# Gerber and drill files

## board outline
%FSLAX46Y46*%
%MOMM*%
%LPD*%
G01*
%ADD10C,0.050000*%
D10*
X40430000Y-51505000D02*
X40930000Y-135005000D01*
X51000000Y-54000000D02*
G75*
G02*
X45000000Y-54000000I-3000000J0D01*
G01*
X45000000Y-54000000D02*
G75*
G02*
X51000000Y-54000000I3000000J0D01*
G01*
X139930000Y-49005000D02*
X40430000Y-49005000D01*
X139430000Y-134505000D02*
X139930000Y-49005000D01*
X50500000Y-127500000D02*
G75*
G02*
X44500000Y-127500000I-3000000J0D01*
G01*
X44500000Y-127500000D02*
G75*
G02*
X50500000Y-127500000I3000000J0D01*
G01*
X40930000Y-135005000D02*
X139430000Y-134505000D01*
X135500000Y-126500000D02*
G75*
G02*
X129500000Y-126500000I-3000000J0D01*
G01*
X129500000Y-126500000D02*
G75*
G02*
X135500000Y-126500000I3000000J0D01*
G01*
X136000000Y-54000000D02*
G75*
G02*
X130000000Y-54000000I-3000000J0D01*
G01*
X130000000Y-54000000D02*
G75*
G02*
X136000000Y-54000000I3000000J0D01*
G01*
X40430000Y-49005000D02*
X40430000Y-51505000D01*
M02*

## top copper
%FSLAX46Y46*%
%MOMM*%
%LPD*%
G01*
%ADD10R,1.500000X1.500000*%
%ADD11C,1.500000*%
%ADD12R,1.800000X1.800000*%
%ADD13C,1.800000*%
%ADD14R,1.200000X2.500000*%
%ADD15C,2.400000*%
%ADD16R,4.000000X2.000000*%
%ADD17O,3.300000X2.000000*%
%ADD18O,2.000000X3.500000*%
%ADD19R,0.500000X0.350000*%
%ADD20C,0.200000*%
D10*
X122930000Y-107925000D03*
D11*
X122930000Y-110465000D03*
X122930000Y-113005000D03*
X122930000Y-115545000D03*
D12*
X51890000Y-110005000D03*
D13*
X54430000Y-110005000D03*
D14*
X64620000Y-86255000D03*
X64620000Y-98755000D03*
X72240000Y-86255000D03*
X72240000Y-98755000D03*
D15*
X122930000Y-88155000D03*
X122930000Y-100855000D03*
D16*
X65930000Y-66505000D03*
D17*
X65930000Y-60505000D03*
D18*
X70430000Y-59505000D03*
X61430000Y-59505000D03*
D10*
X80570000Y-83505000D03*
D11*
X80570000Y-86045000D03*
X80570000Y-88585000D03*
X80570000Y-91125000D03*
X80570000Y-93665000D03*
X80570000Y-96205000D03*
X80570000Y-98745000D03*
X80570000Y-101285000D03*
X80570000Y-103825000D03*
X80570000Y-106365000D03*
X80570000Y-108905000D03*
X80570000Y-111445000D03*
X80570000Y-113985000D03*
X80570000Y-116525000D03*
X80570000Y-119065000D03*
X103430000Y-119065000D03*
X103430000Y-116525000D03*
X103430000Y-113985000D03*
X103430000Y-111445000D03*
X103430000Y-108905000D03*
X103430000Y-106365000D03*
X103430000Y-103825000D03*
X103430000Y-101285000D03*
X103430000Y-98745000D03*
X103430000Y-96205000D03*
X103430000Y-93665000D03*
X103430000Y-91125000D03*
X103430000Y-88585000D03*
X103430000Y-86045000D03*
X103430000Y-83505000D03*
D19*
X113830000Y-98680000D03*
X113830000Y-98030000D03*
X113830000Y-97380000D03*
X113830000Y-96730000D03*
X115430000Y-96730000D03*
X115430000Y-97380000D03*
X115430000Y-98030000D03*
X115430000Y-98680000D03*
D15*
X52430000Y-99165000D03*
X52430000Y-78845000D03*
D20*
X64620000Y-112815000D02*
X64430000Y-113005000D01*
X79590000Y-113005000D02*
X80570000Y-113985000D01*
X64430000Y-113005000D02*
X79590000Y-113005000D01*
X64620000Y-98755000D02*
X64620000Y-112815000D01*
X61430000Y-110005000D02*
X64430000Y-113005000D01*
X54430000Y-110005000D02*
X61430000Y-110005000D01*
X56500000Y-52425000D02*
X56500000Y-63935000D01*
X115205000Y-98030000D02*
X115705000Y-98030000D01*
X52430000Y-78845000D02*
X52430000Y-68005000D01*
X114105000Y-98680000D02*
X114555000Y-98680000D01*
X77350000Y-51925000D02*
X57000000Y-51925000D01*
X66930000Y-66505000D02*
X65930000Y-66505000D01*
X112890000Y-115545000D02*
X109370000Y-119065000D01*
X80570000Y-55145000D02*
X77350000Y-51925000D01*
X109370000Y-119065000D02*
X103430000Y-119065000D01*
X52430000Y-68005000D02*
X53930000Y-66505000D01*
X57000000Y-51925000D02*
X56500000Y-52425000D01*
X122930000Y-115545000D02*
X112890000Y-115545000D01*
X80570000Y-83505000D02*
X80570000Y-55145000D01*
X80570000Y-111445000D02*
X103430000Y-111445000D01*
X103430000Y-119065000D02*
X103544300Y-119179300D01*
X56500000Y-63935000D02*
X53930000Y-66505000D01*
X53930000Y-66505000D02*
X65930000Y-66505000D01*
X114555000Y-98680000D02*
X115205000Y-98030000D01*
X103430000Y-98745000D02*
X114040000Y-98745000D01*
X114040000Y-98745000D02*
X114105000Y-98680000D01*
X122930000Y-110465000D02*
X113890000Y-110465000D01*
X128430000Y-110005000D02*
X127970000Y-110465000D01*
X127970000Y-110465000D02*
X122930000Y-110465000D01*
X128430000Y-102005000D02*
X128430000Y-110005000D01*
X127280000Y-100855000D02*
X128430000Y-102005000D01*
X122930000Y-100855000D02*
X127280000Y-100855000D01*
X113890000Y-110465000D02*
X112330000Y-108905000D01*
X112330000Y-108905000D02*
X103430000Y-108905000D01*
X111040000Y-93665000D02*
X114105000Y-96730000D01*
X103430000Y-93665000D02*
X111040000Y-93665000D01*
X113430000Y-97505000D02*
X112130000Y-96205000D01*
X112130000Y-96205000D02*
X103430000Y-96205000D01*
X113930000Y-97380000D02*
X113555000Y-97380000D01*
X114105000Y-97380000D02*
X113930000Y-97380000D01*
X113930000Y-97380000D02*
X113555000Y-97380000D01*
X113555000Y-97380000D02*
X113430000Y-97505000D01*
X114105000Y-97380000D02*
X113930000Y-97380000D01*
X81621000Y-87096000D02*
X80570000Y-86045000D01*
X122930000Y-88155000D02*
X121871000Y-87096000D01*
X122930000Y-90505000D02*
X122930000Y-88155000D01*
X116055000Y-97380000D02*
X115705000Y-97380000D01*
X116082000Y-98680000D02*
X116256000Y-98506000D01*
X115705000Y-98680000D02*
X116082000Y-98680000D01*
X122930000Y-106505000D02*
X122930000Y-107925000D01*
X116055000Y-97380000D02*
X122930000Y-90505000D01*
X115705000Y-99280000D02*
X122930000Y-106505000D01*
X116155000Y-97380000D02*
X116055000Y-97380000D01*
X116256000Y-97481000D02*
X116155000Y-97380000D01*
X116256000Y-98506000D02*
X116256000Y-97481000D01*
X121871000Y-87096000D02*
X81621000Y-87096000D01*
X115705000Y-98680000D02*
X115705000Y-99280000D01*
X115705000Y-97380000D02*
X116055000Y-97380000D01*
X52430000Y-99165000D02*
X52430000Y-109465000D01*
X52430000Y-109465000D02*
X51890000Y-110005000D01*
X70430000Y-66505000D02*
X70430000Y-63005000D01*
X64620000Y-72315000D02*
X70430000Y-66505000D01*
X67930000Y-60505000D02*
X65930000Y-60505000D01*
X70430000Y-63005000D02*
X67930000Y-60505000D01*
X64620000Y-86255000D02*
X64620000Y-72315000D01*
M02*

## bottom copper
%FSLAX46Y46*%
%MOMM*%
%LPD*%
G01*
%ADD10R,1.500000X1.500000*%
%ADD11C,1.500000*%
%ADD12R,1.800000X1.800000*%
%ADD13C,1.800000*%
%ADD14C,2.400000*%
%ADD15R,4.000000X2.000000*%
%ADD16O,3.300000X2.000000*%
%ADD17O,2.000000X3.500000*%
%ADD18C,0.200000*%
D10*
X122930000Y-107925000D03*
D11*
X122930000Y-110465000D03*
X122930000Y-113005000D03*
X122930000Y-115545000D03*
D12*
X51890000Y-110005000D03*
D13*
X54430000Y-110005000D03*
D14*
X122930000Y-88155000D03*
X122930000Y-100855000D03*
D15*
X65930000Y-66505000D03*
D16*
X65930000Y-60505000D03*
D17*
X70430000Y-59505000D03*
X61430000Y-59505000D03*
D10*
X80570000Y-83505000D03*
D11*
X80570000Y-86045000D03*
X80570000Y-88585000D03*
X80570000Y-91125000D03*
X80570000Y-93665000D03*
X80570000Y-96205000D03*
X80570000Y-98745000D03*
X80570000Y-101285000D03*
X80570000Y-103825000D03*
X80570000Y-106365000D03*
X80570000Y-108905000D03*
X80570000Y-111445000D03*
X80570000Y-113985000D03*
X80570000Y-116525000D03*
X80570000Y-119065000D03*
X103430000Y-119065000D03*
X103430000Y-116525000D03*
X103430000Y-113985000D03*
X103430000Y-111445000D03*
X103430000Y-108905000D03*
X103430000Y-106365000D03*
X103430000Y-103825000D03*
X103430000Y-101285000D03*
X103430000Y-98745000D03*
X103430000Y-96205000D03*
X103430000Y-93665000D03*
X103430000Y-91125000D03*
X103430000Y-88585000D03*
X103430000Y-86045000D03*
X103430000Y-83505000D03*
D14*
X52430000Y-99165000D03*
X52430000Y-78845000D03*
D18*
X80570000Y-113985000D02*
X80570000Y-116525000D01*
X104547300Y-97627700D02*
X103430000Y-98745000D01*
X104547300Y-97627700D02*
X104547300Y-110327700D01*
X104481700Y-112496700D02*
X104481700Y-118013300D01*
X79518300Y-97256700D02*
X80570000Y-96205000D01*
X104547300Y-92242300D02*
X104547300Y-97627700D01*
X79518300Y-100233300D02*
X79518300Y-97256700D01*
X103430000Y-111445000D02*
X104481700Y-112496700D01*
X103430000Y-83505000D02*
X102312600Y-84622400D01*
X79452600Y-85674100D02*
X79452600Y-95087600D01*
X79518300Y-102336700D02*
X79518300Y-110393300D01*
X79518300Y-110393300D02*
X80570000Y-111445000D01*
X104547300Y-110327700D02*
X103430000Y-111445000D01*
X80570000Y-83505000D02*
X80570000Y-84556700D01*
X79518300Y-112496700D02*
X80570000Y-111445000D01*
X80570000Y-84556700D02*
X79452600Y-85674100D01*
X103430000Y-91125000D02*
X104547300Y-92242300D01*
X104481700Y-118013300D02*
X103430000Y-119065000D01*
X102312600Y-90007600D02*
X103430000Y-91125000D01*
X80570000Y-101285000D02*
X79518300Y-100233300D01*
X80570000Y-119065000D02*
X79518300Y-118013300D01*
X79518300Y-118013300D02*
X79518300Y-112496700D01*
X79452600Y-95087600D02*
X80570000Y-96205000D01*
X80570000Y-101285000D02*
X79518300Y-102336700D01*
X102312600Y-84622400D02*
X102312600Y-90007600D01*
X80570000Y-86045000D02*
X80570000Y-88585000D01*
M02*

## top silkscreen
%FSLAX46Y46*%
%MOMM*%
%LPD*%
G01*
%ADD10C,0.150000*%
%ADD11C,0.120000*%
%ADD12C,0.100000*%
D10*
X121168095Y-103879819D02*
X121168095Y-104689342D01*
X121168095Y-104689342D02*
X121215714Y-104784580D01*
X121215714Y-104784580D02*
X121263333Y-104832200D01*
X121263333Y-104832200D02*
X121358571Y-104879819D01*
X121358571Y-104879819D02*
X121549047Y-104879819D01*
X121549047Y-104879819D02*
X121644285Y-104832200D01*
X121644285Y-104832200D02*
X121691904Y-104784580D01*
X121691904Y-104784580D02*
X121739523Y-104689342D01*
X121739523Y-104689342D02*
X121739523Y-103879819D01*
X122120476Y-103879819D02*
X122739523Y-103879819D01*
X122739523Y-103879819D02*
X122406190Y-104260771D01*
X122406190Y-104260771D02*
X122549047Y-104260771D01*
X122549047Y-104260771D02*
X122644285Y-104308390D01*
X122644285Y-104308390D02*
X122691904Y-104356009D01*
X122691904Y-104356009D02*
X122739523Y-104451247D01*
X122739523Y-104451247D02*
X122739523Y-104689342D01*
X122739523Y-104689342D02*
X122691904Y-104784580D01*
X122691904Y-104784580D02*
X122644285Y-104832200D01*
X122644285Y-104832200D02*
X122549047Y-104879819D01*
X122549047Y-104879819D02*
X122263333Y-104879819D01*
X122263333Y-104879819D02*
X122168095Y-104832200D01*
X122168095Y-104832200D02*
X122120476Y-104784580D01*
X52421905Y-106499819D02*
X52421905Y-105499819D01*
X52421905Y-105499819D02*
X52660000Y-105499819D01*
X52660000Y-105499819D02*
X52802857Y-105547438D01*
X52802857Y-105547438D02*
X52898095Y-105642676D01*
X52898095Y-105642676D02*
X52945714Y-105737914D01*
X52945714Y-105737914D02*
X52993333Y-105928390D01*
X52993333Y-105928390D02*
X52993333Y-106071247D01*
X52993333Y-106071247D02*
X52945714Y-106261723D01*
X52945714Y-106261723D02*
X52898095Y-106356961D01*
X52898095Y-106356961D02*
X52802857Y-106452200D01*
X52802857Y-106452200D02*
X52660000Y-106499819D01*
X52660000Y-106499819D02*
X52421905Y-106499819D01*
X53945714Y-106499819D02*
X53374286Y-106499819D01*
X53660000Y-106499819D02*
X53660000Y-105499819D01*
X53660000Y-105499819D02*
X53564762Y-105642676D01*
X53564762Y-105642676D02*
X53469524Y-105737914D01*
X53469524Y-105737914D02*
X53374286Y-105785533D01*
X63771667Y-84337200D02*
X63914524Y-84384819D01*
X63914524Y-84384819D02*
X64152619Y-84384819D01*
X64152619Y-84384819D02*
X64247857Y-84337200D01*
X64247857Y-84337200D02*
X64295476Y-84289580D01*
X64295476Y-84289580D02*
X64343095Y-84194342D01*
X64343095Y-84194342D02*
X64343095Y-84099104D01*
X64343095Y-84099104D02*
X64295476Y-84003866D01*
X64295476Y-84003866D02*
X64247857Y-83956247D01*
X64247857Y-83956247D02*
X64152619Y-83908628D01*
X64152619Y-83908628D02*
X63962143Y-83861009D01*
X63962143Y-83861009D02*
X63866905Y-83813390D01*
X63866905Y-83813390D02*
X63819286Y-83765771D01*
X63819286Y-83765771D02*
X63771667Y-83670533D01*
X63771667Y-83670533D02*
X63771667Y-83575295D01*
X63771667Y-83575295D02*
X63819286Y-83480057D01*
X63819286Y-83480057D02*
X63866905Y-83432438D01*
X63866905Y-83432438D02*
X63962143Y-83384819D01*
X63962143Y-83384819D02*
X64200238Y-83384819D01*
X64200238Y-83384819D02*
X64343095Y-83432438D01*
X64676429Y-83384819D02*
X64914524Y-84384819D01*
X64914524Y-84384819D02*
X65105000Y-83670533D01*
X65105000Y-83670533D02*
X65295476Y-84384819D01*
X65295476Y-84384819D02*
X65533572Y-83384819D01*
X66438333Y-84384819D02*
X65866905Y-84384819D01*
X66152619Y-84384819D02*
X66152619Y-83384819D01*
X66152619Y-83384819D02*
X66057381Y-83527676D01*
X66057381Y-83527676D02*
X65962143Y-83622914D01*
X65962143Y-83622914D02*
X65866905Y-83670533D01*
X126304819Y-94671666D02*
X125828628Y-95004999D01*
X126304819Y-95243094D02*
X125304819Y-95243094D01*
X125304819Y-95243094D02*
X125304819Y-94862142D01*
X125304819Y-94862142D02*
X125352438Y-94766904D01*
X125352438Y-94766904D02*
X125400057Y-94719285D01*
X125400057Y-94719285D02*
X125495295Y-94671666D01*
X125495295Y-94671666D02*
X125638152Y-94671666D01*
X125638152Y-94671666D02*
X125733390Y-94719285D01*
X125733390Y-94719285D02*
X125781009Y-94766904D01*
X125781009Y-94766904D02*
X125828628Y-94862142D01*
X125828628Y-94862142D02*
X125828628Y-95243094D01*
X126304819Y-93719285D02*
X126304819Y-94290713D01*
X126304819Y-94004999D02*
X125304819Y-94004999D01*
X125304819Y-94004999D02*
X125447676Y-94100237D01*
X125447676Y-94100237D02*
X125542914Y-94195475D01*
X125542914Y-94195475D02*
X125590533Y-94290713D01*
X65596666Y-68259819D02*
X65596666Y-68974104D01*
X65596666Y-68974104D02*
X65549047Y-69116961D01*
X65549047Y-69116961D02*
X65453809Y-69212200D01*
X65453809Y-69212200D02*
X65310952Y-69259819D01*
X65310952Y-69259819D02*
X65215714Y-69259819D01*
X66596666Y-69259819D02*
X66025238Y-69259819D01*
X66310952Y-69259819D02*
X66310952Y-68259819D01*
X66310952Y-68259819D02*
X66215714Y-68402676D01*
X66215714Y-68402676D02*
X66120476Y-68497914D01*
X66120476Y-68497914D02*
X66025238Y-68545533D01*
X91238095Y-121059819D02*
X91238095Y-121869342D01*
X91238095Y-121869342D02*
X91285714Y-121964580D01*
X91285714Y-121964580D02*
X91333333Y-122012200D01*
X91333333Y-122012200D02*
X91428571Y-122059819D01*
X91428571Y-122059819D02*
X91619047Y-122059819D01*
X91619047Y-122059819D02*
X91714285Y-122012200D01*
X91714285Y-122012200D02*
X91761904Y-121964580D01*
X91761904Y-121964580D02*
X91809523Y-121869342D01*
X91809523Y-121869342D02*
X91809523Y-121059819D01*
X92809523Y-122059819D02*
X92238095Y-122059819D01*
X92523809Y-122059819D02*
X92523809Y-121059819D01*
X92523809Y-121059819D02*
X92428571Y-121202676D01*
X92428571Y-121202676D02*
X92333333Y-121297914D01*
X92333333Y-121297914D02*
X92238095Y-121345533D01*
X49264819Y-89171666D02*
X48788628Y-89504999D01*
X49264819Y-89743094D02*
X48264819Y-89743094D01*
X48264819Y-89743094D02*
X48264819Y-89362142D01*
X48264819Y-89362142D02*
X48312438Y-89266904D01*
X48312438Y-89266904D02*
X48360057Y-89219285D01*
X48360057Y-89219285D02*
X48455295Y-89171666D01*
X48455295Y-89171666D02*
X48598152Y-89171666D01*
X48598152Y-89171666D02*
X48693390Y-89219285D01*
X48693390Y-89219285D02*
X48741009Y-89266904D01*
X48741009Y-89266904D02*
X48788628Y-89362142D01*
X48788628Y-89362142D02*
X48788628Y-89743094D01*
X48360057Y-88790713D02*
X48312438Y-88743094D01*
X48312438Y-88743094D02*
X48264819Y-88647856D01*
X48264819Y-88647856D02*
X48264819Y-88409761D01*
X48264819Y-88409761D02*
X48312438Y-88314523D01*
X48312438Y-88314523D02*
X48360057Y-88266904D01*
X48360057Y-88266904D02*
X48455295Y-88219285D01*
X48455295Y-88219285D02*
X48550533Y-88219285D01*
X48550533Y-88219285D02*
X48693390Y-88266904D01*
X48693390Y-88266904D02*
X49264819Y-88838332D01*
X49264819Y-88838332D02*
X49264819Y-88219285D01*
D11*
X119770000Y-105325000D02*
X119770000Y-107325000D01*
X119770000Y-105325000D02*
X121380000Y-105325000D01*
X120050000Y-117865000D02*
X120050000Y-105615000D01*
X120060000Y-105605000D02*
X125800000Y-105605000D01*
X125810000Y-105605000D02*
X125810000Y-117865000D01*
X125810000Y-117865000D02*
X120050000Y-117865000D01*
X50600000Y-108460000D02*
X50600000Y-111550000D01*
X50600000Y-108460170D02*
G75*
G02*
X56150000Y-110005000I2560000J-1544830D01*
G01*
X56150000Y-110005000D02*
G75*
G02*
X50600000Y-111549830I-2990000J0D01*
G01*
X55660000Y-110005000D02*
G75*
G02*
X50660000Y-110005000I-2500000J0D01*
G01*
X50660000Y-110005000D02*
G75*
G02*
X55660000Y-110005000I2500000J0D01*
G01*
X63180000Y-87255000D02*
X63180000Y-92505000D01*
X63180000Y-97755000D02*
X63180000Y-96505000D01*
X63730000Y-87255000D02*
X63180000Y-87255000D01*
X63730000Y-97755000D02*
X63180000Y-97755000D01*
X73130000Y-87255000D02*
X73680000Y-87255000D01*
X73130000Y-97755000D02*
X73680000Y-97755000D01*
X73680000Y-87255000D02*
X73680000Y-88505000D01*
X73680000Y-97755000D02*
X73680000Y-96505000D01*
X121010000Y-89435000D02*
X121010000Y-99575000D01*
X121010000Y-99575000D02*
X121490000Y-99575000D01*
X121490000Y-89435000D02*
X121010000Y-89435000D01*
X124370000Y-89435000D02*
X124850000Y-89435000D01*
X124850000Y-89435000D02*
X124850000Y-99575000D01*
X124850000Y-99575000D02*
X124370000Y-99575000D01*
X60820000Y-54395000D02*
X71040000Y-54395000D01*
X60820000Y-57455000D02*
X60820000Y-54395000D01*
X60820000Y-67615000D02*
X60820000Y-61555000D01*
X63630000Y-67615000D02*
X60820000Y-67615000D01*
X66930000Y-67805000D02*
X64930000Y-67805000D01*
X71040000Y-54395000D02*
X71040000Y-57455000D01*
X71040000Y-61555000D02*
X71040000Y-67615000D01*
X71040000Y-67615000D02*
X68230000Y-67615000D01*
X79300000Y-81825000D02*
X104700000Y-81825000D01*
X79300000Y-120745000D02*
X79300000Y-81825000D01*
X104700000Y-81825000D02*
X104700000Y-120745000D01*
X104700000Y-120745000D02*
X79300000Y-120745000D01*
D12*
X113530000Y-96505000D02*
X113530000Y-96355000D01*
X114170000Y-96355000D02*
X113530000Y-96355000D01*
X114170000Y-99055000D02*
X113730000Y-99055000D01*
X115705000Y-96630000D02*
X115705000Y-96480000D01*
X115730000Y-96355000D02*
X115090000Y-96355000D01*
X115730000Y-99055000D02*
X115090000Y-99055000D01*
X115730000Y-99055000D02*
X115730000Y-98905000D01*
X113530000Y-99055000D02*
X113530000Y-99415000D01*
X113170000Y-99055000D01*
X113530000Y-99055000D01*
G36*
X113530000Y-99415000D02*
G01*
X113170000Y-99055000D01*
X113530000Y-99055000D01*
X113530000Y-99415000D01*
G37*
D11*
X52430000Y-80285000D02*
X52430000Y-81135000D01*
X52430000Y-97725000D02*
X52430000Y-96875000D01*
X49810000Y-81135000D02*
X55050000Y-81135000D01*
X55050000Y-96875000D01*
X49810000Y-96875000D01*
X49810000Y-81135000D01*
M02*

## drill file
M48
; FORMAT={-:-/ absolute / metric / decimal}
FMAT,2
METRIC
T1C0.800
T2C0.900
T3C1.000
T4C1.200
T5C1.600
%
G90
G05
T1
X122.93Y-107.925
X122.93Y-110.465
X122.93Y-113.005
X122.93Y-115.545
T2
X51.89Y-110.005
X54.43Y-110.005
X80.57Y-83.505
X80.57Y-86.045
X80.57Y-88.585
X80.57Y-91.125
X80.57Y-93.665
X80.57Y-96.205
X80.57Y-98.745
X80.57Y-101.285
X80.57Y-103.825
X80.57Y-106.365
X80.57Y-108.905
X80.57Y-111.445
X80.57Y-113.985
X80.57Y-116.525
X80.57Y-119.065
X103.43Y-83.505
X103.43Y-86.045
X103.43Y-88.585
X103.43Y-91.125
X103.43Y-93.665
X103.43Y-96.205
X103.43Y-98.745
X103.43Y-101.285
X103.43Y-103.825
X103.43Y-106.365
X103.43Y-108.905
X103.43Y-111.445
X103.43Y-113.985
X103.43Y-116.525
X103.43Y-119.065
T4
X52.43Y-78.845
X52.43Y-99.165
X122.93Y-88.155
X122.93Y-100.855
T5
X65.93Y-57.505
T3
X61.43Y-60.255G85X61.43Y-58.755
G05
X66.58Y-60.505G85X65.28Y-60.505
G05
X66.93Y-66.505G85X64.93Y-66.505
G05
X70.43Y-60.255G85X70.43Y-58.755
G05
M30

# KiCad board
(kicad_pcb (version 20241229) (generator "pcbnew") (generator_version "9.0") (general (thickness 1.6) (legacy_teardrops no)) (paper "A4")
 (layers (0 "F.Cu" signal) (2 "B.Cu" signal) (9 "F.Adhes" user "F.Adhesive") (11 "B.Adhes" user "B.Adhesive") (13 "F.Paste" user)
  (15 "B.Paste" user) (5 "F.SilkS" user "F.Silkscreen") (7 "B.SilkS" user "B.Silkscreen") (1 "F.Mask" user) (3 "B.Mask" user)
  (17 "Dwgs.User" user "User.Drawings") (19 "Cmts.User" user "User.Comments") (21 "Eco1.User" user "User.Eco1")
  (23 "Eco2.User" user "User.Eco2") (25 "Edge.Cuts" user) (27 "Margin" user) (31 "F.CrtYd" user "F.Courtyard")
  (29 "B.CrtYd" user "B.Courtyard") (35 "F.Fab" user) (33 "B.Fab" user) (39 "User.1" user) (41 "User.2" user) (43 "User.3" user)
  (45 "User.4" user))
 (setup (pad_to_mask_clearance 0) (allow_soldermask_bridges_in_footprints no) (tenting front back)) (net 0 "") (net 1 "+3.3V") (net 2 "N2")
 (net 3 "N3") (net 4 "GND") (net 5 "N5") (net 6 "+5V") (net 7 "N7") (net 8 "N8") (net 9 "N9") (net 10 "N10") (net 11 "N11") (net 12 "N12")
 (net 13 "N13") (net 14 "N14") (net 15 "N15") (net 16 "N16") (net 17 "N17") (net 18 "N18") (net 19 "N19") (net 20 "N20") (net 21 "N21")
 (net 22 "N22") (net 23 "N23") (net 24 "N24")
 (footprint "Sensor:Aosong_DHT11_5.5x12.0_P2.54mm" (layer "F.Cu") (at 122.93 107.925)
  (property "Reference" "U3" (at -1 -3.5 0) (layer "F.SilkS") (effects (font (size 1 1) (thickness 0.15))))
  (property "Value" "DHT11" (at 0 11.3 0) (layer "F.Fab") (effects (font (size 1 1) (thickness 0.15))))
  (fp_line (start -3.16 -2.6) (end -3.16 -0.6) (stroke (width 0.12) (type solid)) (layer "F.SilkS"))
  (fp_line (start -3.16 -2.6) (end -1.55 -2.6) (stroke (width 0.12) (type solid)) (layer "F.SilkS"))
  (fp_line (start -2.88 9.94) (end -2.88 -2.31) (stroke (width 0.12) (type solid)) (layer "F.SilkS"))
  (fp_line (start -2.87 -2.32) (end 2.87 -2.32) (stroke (width 0.12) (type solid)) (layer "F.SilkS"))
  (fp_line (start 2.88 -2.32) (end 2.88 9.94) (stroke (width 0.12) (type solid)) (layer "F.SilkS"))
  (fp_line (start 2.88 9.94) (end -2.88 9.94) (stroke (width 0.12) (type solid)) (layer "F.SilkS"))
  (pad "1" thru_hole rect (at 0 0) (size 1.5 1.5) (drill 0.8) (layers "*.Cu" "*.Mask") (remove_unused_layers no) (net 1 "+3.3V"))
  (pad "2" thru_hole circle (at 0 2.54) (size 1.5 1.5) (drill 0.8) (layers "*.Cu" "*.Mask") (remove_unused_layers no) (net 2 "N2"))
  (pad "3" thru_hole circle (at 0 5.08) (size 1.5 1.5) (drill 0.8) (layers "*.Cu" "*.Mask") (remove_unused_layers no) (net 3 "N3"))
  (pad "4" thru_hole circle (at 0 7.62) (size 1.5 1.5) (drill 0.8) (layers "*.Cu" "*.Mask") (remove_unused_layers no) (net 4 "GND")))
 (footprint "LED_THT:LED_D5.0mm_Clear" (layer "F.Cu") (at 51.89 110.005)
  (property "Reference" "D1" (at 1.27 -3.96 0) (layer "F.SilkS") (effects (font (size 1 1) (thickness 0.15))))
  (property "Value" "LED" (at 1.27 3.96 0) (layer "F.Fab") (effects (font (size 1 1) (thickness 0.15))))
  (fp_line (start -1.29 -1.545) (end -1.29 1.545) (stroke (width 0.12) (type solid)) (layer "F.SilkS"))
  (fp_arc (start -1.29 -1.54483) (mid 2.071779 -2.880495) (end 4.26 0) (stroke (width 0.12) (type solid)) (layer "F.SilkS"))
  (fp_arc (start 4.26 0) (mid 2.071779 2.880495) (end -1.29 1.54483) (stroke (width 0.12) (type solid)) (layer "F.SilkS"))
  (fp_circle (center 1.27 0) (end 3.77 0) (stroke (width 0.12) (type solid)) (fill no) (layer "F.SilkS"))
  (pad "1" thru_hole rect (at 0 0) (size 1.8 1.8) (drill 0.9) (layers "*.Cu" "*.Mask") (remove_unused_layers no) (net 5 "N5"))
  (pad "2" thru_hole circle (at 2.54 0) (size 1.8 1.8) (drill 0.9) (layers "*.Cu" "*.Mask") (remove_unused_layers no) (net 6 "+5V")))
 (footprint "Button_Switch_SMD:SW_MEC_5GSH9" (layer "F.Cu") (at 68.43 92.505)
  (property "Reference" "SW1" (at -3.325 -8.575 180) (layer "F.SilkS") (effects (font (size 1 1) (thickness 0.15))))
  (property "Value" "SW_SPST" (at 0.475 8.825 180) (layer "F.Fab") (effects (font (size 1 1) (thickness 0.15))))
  (fp_line (start -5.25 -5.25) (end -5.25 0) (stroke (width 0.12) (type solid)) (layer "F.SilkS"))
  (fp_line (start -5.25 5.25) (end -5.25 4) (stroke (width 0.12) (type solid)) (layer "F.SilkS"))
  (fp_line (start -4.7 -5.25) (end -5.25 -5.25) (stroke (width 0.12) (type solid)) (layer "F.SilkS"))
  (fp_line (start -4.7 5.25) (end -5.25 5.25) (stroke (width 0.12) (type solid)) (layer "F.SilkS"))
  (fp_line (start 4.7 -5.25) (end 5.25 -5.25) (stroke (width 0.12) (type solid)) (layer "F.SilkS"))
  (fp_line (start 4.7 5.25) (end 5.25 5.25) (stroke (width 0.12) (type solid)) (layer "F.SilkS"))
  (fp_line (start 5.25 -5.25) (end 5.25 -4) (stroke (width 0.12) (type solid)) (layer "F.SilkS"))
  (fp_line (start 5.25 5.25) (end 5.25 4) (stroke (width 0.12) (type solid)) (layer "F.SilkS"))
  (pad "1" smd rect (at -3.81 -6.25 90) (size 2.5 1.2) (layers "F.Cu" "F.Mask" "F.Paste") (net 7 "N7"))
  (pad "2" smd rect (at -3.81 6.25 90) (size 2.5 1.2) (layers "F.Cu" "F.Mask" "F.Paste") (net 6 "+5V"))
  (pad "3" smd rect (at 3.81 -6.25 90) (size 2.5 1.2) (layers "F.Cu" "F.Mask" "F.Paste"))
  (pad "4" smd rect (at 3.81 6.25 90) (size 2.5 1.2) (layers "F.Cu" "F.Mask" "F.Paste")))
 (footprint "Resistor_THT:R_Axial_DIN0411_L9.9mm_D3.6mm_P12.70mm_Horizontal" (layer "F.Cu") (at 122.93 88.155 -90)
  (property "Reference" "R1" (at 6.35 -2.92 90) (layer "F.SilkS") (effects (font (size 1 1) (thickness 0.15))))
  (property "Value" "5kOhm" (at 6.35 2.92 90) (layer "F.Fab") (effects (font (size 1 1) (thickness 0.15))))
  (fp_line (start 1.28 1.92) (end 11.42 1.92) (stroke (width 0.12) (type solid)) (layer "F.SilkS"))
  (fp_line (start 11.42 1.92) (end 11.42 1.44) (stroke (width 0.12) (type solid)) (layer "F.SilkS"))
  (fp_line (start 1.28 1.44) (end 1.28 1.92) (stroke (width 0.12) (type solid)) (layer "F.SilkS"))
  (fp_line (start 1.28 -1.44) (end 1.28 -1.92) (stroke (width 0.12) (type solid)) (layer "F.SilkS"))
  (fp_line (start 1.28 -1.92) (end 11.42 -1.92) (stroke (width 0.12) (type solid)) (layer "F.SilkS"))
  (fp_line (start 11.42 -1.92) (end 11.42 -1.44) (stroke (width 0.12) (type solid)) (layer "F.SilkS"))
  (pad "1" thru_hole circle (at 0 0 270) (size 2.4 2.4) (drill 1.2) (layers "*.Cu" "*.Mask") (remove_unused_layers no) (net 1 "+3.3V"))
  (pad "2" thru_hole circle (at 12.7 0 270) (size 2.4 2.4) (drill 1.2) (layers "*.Cu" "*.Mask") (remove_unused_layers no) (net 2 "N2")))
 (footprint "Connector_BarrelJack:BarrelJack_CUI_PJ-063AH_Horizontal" (layer "F.Cu") (at 65.93 66.505 180)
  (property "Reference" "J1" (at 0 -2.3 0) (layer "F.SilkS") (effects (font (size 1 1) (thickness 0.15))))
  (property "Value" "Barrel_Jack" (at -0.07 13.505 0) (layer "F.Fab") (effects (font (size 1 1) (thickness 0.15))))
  (fp_line (start 5.11 12.11) (end -5.11 12.11) (stroke (width 0.12) (type solid)) (layer "F.SilkS"))
  (fp_line (start 5.11 9.05) (end 5.11 12.11) (stroke (width 0.12) (type solid)) (layer "F.SilkS"))
  (fp_line (start 5.11 -1.11) (end 5.11 4.95) (stroke (width 0.12) (type solid)) (layer "F.SilkS"))
  (fp_line (start 2.3 -1.11) (end 5.11 -1.11) (stroke (width 0.12) (type solid)) (layer "F.SilkS"))
  (fp_line (start -1 -1.3) (end 1 -1.3) (stroke (width 0.12) (type solid)) (layer "F.SilkS"))
  (fp_line (start -5.11 12.11) (end -5.11 9.05) (stroke (width 0.12) (type solid)) (layer "F.SilkS"))
  (fp_line (start -5.11 4.95) (end -5.11 -1.11) (stroke (width 0.12) (type solid)) (layer "F.SilkS"))
  (fp_line (start -5.11 -1.11) (end -2.3 -1.11) (stroke (width 0.12) (type solid)) (layer "F.SilkS"))
  (pad "" np_thru_hole circle (at 0 9 180) (size 1.6 1.6) (drill 1.6) (layers "*.Cu" "*.Mask"))
  (pad "1" thru_hole rect (at 0 0 180) (size 4 2) (drill oval 3 1) (layers "*.Cu" "*.Mask") (remove_unused_layers no) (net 4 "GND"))
  (pad "2" thru_hole oval (at 0 6 180) (size 3.3 2) (drill oval 2.3 1) (layers "*.Cu" "*.Mask") (remove_unused_layers no) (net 7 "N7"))
  (pad "MP" thru_hole oval (at -4.5 7 180) (size 2 3.5) (drill oval 1 2.5) (layers "*.Cu" "*.Mask") (remove_unused_layers no))
  (pad "MP" thru_hole oval (at 4.5 7 180) (size 2 3.5) (drill oval 1 2.5) (layers "*.Cu" "*.Mask") (remove_unused_layers no)))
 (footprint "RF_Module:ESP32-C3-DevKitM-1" (layer "F.Cu") (at 80.57 83.505)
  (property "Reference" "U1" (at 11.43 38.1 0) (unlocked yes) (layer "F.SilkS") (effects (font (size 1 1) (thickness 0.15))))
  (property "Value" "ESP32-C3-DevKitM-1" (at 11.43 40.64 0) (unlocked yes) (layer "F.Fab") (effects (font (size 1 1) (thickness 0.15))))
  (fp_line (start -1.27 -1.68) (end 24.13 -1.68) (stroke (width 0.12) (type solid)) (layer "F.SilkS"))
  (fp_line (start -1.27 37.24) (end -1.27 -1.68) (stroke (width 0.12) (type solid)) (layer "F.SilkS"))
  (fp_line (start 24.13 -1.68) (end 24.13 37.24) (stroke (width 0.12) (type solid)) (layer "F.SilkS"))
  (fp_line (start 24.13 37.24) (end -1.27 37.24) (stroke (width 0.12) (type solid)) (layer "F.SilkS"))
  (pad "1" thru_hole rect (at 0 0) (size 1.5 1.5) (drill 0.9) (layers "*.Cu" "*.Mask") (remove_unused_layers yes) (keep_end_layers yes)
   (zone_layer_connections) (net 4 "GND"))
  (pad "2" thru_hole circle (at 0 2.54) (size 1.5 1.5) (drill 0.9) (layers "*.Cu" "*.Mask") (remove_unused_layers yes) (keep_end_layers yes)
   (zone_layer_connections) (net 1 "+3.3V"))
  (pad "3" thru_hole circle (at 0 5.08) (size 1.5 1.5) (drill 0.9) (layers "*.Cu" "*.Mask") (remove_unused_layers yes) (keep_end_layers yes)
   (zone_layer_connections) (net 1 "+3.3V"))
  (pad "4" thru_hole circle (at 0 7.62) (size 1.5 1.5) (drill 0.9) (layers "*.Cu" "*.Mask") (remove_unused_layers yes) (keep_end_layers yes)
   (zone_layer_connections) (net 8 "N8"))
  (pad "5" thru_hole circle (at 0 10.16) (size 1.5 1.5) (drill 0.9) (layers "*.Cu" "*.Mask") (remove_unused_layers yes)
   (keep_end_layers yes) (zone_layer_connections) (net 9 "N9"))
  (pad "6" thru_hole circle (at 0 12.7) (size 1.5 1.5) (drill 0.9) (layers "*.Cu" "*.Mask") (remove_unused_layers yes) (keep_end_layers yes)
   (zone_layer_connections) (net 4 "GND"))
  (pad "7" thru_hole circle (at 0 15.24) (size 1.5 1.5) (drill 0.9) (layers "*.Cu" "*.Mask") (remove_unused_layers yes)
   (keep_end_layers yes) (zone_layer_connections) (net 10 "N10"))
  (pad "8" thru_hole circle (at 0 17.78) (size 1.5 1.5) (drill 0.9) (layers "*.Cu" "*.Mask") (remove_unused_layers yes)
   (keep_end_layers yes) (zone_layer_connections) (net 4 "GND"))
  (pad "9" thru_hole circle (at 0 20.32) (size 1.5 1.5) (drill 0.9) (layers "*.Cu" "*.Mask") (remove_unused_layers yes)
   (keep_end_layers yes) (zone_layer_connections) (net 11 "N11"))
  (pad "10" thru_hole circle (at 0 22.86) (size 1.5 1.5) (drill 0.9) (layers "*.Cu" "*.Mask") (remove_unused_layers yes)
   (keep_end_layers yes) (zone_layer_connections) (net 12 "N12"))
  (pad "11" thru_hole circle (at 0 25.4) (size 1.5 1.5) (drill 0.9) (layers "*.Cu" "*.Mask") (remove_unused_layers yes)
   (keep_end_layers yes) (zone_layer_connections) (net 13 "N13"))
  (pad "12" thru_hole circle (at 0 27.94) (size 1.5 1.5) (drill 0.9) (layers "*.Cu" "*.Mask") (remove_unused_layers yes)
   (keep_end_layers yes) (zone_layer_connections) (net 4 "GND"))
  (pad "13" thru_hole circle (at 0 30.48) (size 1.5 1.5) (drill 0.9) (layers "*.Cu" "*.Mask") (remove_unused_layers yes)
   (keep_end_layers yes) (zone_layer_connections) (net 6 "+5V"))
  (pad "14" thru_hole circle (at 0 33.02) (size 1.5 1.5) (drill 0.9) (layers "*.Cu" "*.Mask") (remove_unused_layers yes)
   (keep_end_layers yes) (zone_layer_connections) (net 6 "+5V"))
  (pad "15" thru_hole circle (at 0 35.56) (size 1.5 1.5) (drill 0.9) (layers "*.Cu" "*.Mask") (remove_unused_layers yes)
   (keep_end_layers yes) (zone_layer_connections) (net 4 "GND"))
  (pad "16" thru_hole circle (at 22.86 35.56) (size 1.5 1.5) (drill 0.9) (layers "*.Cu" "*.Mask") (remove_unused_layers yes)
   (keep_end_layers yes) (zone_layer_connections) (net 4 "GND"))
  (pad "17" thru_hole circle (at 22.86 33.02) (size 1.5 1.5) (drill 0.9) (layers "*.Cu" "*.Mask") (remove_unused_layers yes)
   (keep_end_layers yes) (zone_layer_connections) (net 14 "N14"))
  (pad "18" thru_hole circle (at 22.86 30.48) (size 1.5 1.5) (drill 0.9) (layers "*.Cu" "*.Mask") (remove_unused_layers yes)
   (keep_end_layers yes) (zone_layer_connections) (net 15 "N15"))
  (pad "19" thru_hole circle (at 22.86 27.94) (size 1.5 1.5) (drill 0.9) (layers "*.Cu" "*.Mask") (remove_unused_layers yes)
   (keep_end_layers yes) (zone_layer_connections) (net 4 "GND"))
  (pad "20" thru_hole circle (at 22.86 25.4) (size 1.5 1.5) (drill 0.9) (layers "*.Cu" "*.Mask") (remove_unused_layers yes)
   (keep_end_layers yes) (zone_layer_connections) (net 2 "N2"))
  (pad "21" thru_hole circle (at 22.86 22.86) (size 1.5 1.5) (drill 0.9) (layers "*.Cu" "*.Mask") (remove_unused_layers yes)
   (keep_end_layers yes) (zone_layer_connections) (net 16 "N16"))
  (pad "22" thru_hole circle (at 22.86 20.32) (size 1.5 1.5) (drill 0.9) (layers "*.Cu" "*.Mask") (remove_unused_layers yes)
   (keep_end_layers yes) (zone_layer_connections) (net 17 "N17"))
  (pad "23" thru_hole circle (at 22.86 17.78) (size 1.5 1.5) (drill 0.9) (layers "*.Cu" "*.Mask") (remove_unused_layers yes)
   (keep_end_layers yes) (zone_layer_connections) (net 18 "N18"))
  (pad "24" thru_hole circle (at 22.86 15.24) (size 1.5 1.5) (drill 0.9) (layers "*.Cu" "*.Mask") (remove_unused_layers yes)
   (keep_end_layers yes) (zone_layer_connections) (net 4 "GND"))
  (pad "25" thru_hole circle (at 22.86 12.7) (size 1.5 1.5) (drill 0.9) (layers "*.Cu" "*.Mask") (remove_unused_layers yes)
   (keep_end_layers yes) (zone_layer_connections) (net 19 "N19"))
  (pad "26" thru_hole circle (at 22.86 10.16) (size 1.5 1.5) (drill 0.9) (layers "*.Cu" "*.Mask") (remove_unused_layers yes)
   (keep_end_layers yes) (zone_layer_connections) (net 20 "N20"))
  (pad "27" thru_hole circle (at 22.86 7.62) (size 1.5 1.5) (drill 0.9) (layers "*.Cu" "*.Mask") (remove_unused_layers yes)
   (keep_end_layers yes) (zone_layer_connections) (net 4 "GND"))
  (pad "28" thru_hole circle (at 22.86 5.08) (size 1.5 1.5) (drill 0.9) (layers "*.Cu" "*.Mask") (remove_unused_layers yes)
   (keep_end_layers yes) (zone_layer_connections) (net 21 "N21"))
  (pad "29" thru_hole circle (at 22.86 2.54) (size 1.5 1.5) (drill 0.9) (layers "*.Cu" "*.Mask") (remove_unused_layers yes)
   (keep_end_layers yes) (zone_layer_connections) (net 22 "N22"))
  (pad "30" thru_hole circle (at 22.86 0) (size 1.5 1.5) (drill 0.9) (layers "*.Cu" "*.Mask") (remove_unused_layers yes)
   (keep_end_layers yes) (zone_layer_connections) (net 4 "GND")))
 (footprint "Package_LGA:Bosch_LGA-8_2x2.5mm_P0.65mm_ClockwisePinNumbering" (layer "F.Cu") (at 114.63 97.705 90)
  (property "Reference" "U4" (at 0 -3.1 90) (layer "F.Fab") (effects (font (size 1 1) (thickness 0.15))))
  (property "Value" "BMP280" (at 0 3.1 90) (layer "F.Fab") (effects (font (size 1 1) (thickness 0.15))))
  (fp_line (start 1.2 -1.1) (end 1.35 -1.1) (stroke (width 0.1) (type solid)) (layer "F.SilkS"))
  (fp_line (start 1.35 -0.46) (end 1.35 -1.1) (stroke (width 0.1) (type solid)) (layer "F.SilkS"))
  (fp_line (start -1.35 -0.46) (end -1.35 -0.9) (stroke (width 0.1) (type solid)) (layer "F.SilkS"))
  (fp_line (start 1.075 1.075) (end 1.225 1.075) (stroke (width 0.1) (type solid)) (layer "F.SilkS"))
  (fp_line (start 1.35 1.1) (end 1.35 0.46) (stroke (width 0.1) (type solid)) (layer "F.SilkS"))
  (fp_line (start -1.35 1.1) (end -1.35 0.46) (stroke (width 0.1) (type solid)) (layer "F.SilkS"))
  (fp_line (start -1.35 1.1) (end -1.2 1.1) (stroke (width 0.1) (type solid)) (layer "F.SilkS"))
  (fp_poly
   (pts (xy -1.35 -1.1) (xy -1.71 -1.1) (xy -1.35 -1.46) (xy -1.35 -1.1)) (stroke (width 0.1) (type solid)) (fill yes) (layer "F.SilkS"))
  (pad "1" smd rect (at -0.975 -0.8 180) (size 0.5 0.35) (layers "F.Cu" "F.Mask" "F.Paste") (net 4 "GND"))
  (pad "2" smd rect (at -0.325 -0.8 180) (size 0.5 0.35) (layers "F.Cu" "F.Mask" "F.Paste") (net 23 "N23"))
  (pad "3" smd rect (at 0.325 -0.8 180) (size 0.5 0.35) (layers "F.Cu" "F.Mask" "F.Paste") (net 19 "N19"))
  (pad "4" smd rect (at 0.975 -0.8 180) (size 0.5 0.35) (layers "F.Cu" "F.Mask" "F.Paste") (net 20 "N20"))
  (pad "5" smd rect (at 0.975 0.8 180) (size 0.5 0.35) (layers "F.Cu" "F.Mask" "F.Paste") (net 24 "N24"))
  (pad "6" smd rect (at 0.325 0.8 180) (size 0.5 0.35) (layers "F.Cu" "F.Mask" "F.Paste") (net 1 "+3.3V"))
  (pad "7" smd rect (at -0.325 0.8 180) (size 0.5 0.35) (layers "F.Cu" "F.Mask" "F.Paste") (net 4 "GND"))
  (pad "8" smd rect (at -0.975 0.8 180) (size 0.5 0.35) (layers "F.Cu" "F.Mask" "F.Paste") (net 1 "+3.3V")))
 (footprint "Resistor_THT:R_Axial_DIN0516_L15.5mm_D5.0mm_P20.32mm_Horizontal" (layer "F.Cu") (at 52.43 99.165 90)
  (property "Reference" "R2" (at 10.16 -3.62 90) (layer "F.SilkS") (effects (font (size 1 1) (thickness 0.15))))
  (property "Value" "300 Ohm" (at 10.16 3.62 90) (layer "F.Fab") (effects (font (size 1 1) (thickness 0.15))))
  (fp_line (start 18.88 0) (end 18.03 0) (stroke (width 0.12) (type solid)) (layer "F.SilkS"))
  (fp_line (start 1.44 0) (end 2.29 0) (stroke (width 0.12) (type solid)) (layer "F.SilkS"))
  (fp_rect (start 2.29 -2.62) (end 18.03 2.62) (stroke (width 0.12) (type solid)) (fill no) (layer "F.SilkS"))
  (pad "1" thru_hole circle (at 0 0 90) (size 2.4 2.4) (drill 1.2) (layers "*.Cu" "*.Mask") (remove_unused_layers no) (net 5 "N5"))
  (pad "2" thru_hole circle (at 20.32 0 90) (size 2.4 2.4) (drill 1.2) (layers "*.Cu" "*.Mask") (remove_unused_layers no) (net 4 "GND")))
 (gr_line (start 40.43 51.505) (end 40.93 135.005) (stroke (width 0.05) (type default)) (layer "Edge.Cuts"))
 (gr_circle (center 48 54) (end 51 54) (stroke (width 0.05) (type solid)) (fill no) (layer "Edge.Cuts"))
 (gr_line (start 139.93 49.005) (end 40.43 49.005) (stroke (width 0.05) (type default)) (layer "Edge.Cuts"))
 (gr_line (start 139.43 134.505) (end 139.93 49.005) (stroke (width 0.05) (type default)) (layer "Edge.Cuts"))
 (gr_circle (center 47.5 127.5) (end 50.5 127.5) (stroke (width 0.05) (type solid)) (fill no) (layer "Edge.Cuts"))
 (gr_line (start 40.93 135.005) (end 139.43 134.505) (stroke (width 0.05) (type default)) (layer "Edge.Cuts"))
 (gr_circle (center 132.5 126.5) (end 135.5 126.5) (stroke (width 0.05) (type solid)) (fill no) (layer "Edge.Cuts"))
 (gr_circle (center 133 54) (end 136 54) (stroke (width 0.05) (type solid)) (fill no) (layer "Edge.Cuts"))
 (gr_line (start 40.43 49.005) (end 40.43 51.505) (stroke (width 0.05) (type default)) (layer "Edge.Cuts"))
 (segment (start 64.62 112.815) (end 64.43 113.005) (width 0.2) (layer "F.Cu") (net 6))
 (segment (start 79.59 113.005) (end 80.57 113.985) (width 0.2) (layer "F.Cu") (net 6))
 (segment (start 64.43 113.005) (end 79.59 113.005) (width 0.2) (layer "F.Cu") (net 6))
 (segment (start 64.62 98.755) (end 64.62 112.815) (width 0.2) (layer "F.Cu") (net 6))
 (segment (start 61.43 110.005) (end 64.43 113.005) (width 0.2) (layer "F.Cu") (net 6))
 (segment (start 54.43 110.005) (end 61.43 110.005) (width 0.2) (layer "F.Cu") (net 6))
 (segment (start 80.57 113.985) (end 80.57 116.525) (width 0.2) (layer "B.Cu") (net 6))
 (segment (start 56.5 52.425) (end 56.5 63.935) (width 0.2) (layer "F.Cu") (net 4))
 (segment (start 115.205 98.03) (end 115.705 98.03) (width 0.2) (layer "F.Cu") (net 4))
 (segment (start 52.43 78.845) (end 52.43 68.005) (width 0.2) (layer "F.Cu") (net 4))
 (segment (start 114.105 98.68) (end 114.555 98.68) (width 0.2) (layer "F.Cu") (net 4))
 (segment (start 77.35 51.925) (end 57 51.925) (width 0.2) (layer "F.Cu") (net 4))
 (segment (start 66.93 66.505) (end 65.93 66.505) (width 0.2) (layer "F.Cu") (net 4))
 (segment (start 112.89 115.545) (end 109.37 119.065) (width 0.2) (layer "F.Cu") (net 4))
 (segment (start 80.57 55.145) (end 77.35 51.925) (width 0.2) (layer "F.Cu") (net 4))
 (segment (start 109.37 119.065) (end 103.43 119.065) (width 0.2) (layer "F.Cu") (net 4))
 (segment (start 52.43 68.005) (end 53.93 66.505) (width 0.2) (layer "F.Cu") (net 4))
 (segment (start 57 51.925) (end 56.5 52.425) (width 0.2) (layer "F.Cu") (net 4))
 (segment (start 122.93 115.545) (end 112.89 115.545) (width 0.2) (layer "F.Cu") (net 4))
 (segment (start 80.57 83.505) (end 80.57 55.145) (width 0.2) (layer "F.Cu") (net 4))
 (segment (start 80.57 111.445) (end 103.43 111.445) (width 0.2) (layer "F.Cu") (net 4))
 (segment (start 103.43 119.065) (end 103.5443 119.1793) (width 0.2) (layer "F.Cu") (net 4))
 (segment (start 56.5 63.935) (end 53.93 66.505) (width 0.2) (layer "F.Cu") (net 4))
 (segment (start 53.93 66.505) (end 65.93 66.505) (width 0.2) (layer "F.Cu") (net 4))
 (segment (start 114.555 98.68) (end 115.205 98.03) (width 0.2) (layer "F.Cu") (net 4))
 (segment (start 103.43 98.745) (end 114.04 98.745) (width 0.2) (layer "F.Cu") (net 4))
 (segment (start 114.04 98.745) (end 114.105 98.68) (width 0.2) (layer "F.Cu") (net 4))
 (segment (start 104.5473 97.6277) (end 103.43 98.745) (width 0.2) (layer "B.Cu") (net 4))
 (segment (start 104.5473 97.6277) (end 104.5473 110.3277) (width 0.2) (layer "B.Cu") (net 4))
 (segment (start 104.4817 112.4967) (end 104.4817 118.0133) (width 0.2) (layer "B.Cu") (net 4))
 (segment (start 79.5183 97.2567) (end 80.57 96.205) (width 0.2) (layer "B.Cu") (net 4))
 (segment (start 104.5473 92.2423) (end 104.5473 97.6277) (width 0.2) (layer "B.Cu") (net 4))
 (segment (start 79.5183 100.2333) (end 79.5183 97.2567) (width 0.2) (layer "B.Cu") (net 4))
 (segment (start 103.43 111.445) (end 104.4817 112.4967) (width 0.2) (layer "B.Cu") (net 4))
 (segment (start 103.43 83.505) (end 102.3126 84.6224) (width 0.2) (layer "B.Cu") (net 4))
 (segment (start 79.4526 85.6741) (end 79.4526 95.0876) (width 0.2) (layer "B.Cu") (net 4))
 (segment (start 79.5183 102.3367) (end 79.5183 110.3933) (width 0.2) (layer "B.Cu") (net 4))
 (segment (start 79.5183 110.3933) (end 80.57 111.445) (width 0.2) (layer "B.Cu") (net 4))
 (segment (start 104.5473 110.3277) (end 103.43 111.445) (width 0.2) (layer "B.Cu") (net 4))
 (segment (start 80.57 83.505) (end 80.57 84.5567) (width 0.2) (layer "B.Cu") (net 4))
 (segment (start 79.5183 112.4967) (end 80.57 111.445) (width 0.2) (layer "B.Cu") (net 4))
 (segment (start 80.57 84.5567) (end 79.4526 85.6741) (width 0.2) (layer "B.Cu") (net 4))
 (segment (start 103.43 91.125) (end 104.5473 92.2423) (width 0.2) (layer "B.Cu") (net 4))
 (segment (start 104.4817 118.0133) (end 103.43 119.065) (width 0.2) (layer "B.Cu") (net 4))
 (segment (start 102.3126 90.0076) (end 103.43 91.125) (width 0.2) (layer "B.Cu") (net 4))
 (segment (start 80.57 101.285) (end 79.5183 100.2333) (width 0.2) (layer "B.Cu") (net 4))
 (segment (start 80.57 119.065) (end 79.5183 118.0133) (width 0.2) (layer "B.Cu") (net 4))
 (segment (start 79.5183 118.0133) (end 79.5183 112.4967) (width 0.2) (layer "B.Cu") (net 4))
 (segment (start 79.4526 95.0876) (end 80.57 96.205) (width 0.2) (layer "B.Cu") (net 4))
 (segment (start 80.57 101.285) (end 79.5183 102.3367) (width 0.2) (layer "B.Cu") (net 4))
 (segment (start 102.3126 84.6224) (end 102.3126 90.0076) (width 0.2) (layer "B.Cu") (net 4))
 (segment (start 122.93 110.465) (end 113.89 110.465) (width 0.2) (layer "F.Cu") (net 2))
 (segment (start 128.43 110.005) (end 127.97 110.465) (width 0.2) (layer "F.Cu") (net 2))
 (segment (start 127.97 110.465) (end 122.93 110.465) (width 0.2) (layer "F.Cu") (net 2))
 (segment (start 128.43 102.005) (end 128.43 110.005) (width 0.2) (layer "F.Cu") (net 2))
 (segment (start 127.28 100.855) (end 128.43 102.005) (width 0.2) (layer "F.Cu") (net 2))
 (segment (start 122.93 100.855) (end 127.28 100.855) (width 0.2) (layer "F.Cu") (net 2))
 (segment (start 113.89 110.465) (end 112.33 108.905) (width 0.2) (layer "F.Cu") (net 2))
 (segment (start 112.33 108.905) (end 103.43 108.905) (width 0.2) (layer "F.Cu") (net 2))
 (segment (start 111.04 93.665) (end 114.105 96.73) (width 0.2) (layer "F.Cu") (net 20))
 (segment (start 103.43 93.665) (end 111.04 93.665) (width 0.2) (layer "F.Cu") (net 20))
 (segment (start 113.43 97.505) (end 112.13 96.205) (width 0.2) (layer "F.Cu") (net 19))
 (segment (start 112.13 96.205) (end 103.43 96.205) (width 0.2) (layer "F.Cu") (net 19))
 (segment (start 113.93 97.38) (end 113.555 97.38) (width 0.2) (layer "F.Cu") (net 19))
 (segment (start 114.105 97.38) (end 113.93 97.38) (width 0.2) (layer "F.Cu") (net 19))
 (segment (start 113.93 97.38) (end 113.555 97.38) (width 0.2) (layer "F.Cu") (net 19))
 (segment (start 113.555 97.38) (end 113.43 97.505) (width 0.2) (layer "F.Cu") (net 19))
 (segment (start 114.105 97.38) (end 113.93 97.38) (width 0.2) (layer "F.Cu") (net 19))
 (segment (start 81.621 87.096) (end 80.57 86.045) (width 0.2) (layer "F.Cu") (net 1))
 (segment (start 122.93 88.155) (end 121.871 87.096) (width 0.2) (layer "F.Cu") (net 1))
 (segment (start 122.93 90.505) (end 122.93 88.155) (width 0.2) (layer "F.Cu") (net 1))
 (segment (start 116.055 97.38) (end 115.705 97.38) (width 0.2) (layer "F.Cu") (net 1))
 (segment (start 116.082 98.68) (end 116.256 98.506) (width 0.2) (layer "F.Cu") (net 1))
 (segment (start 115.705 98.68) (end 116.082 98.68) (width 0.2) (layer "F.Cu") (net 1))
 (segment (start 122.93 106.505) (end 122.93 107.925) (width 0.2) (layer "F.Cu") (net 1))
 (segment (start 116.055 97.38) (end 122.93 90.505) (width 0.2) (layer "F.Cu") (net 1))
 (segment (start 115.705 99.28) (end 122.93 106.505) (width 0.2) (layer "F.Cu") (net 1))
 (segment (start 116.155 97.38) (end 116.055 97.38) (width 0.2) (layer "F.Cu") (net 1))
 (segment (start 116.256 97.481) (end 116.155 97.38) (width 0.2) (layer "F.Cu") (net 1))
 (segment (start 116.256 98.506) (end 116.256 97.481) (width 0.2) (layer "F.Cu") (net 1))
 (segment (start 121.871 87.096) (end 81.621 87.096) (width 0.2) (layer "F.Cu") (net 1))
 (segment (start 115.705 98.68) (end 115.705 99.28) (width 0.2) (layer "F.Cu") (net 1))
 (segment (start 115.705 97.38) (end 116.055 97.38) (width 0.2) (layer "F.Cu") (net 1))
 (segment (start 80.57 86.045) (end 80.57 88.585) (width 0.2) (layer "B.Cu") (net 1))
 (segment (start 52.43 99.165) (end 52.43 109.465) (width 0.2) (layer "F.Cu") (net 5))
 (segment (start 52.43 109.465) (end 51.89 110.005) (width 0.2) (layer "F.Cu") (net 5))
 (segment (start 70.43 66.505) (end 70.43 63.005) (width 0.2) (layer "F.Cu") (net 7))
 (segment (start 64.62 72.315) (end 70.43 66.505) (width 0.2) (layer "F.Cu") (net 7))
 (segment (start 67.93 60.505) (end 65.93 60.505) (width 0.2) (layer "F.Cu") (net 7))
 (segment (start 70.43 63.005) (end 67.93 60.505) (width 0.2) (layer "F.Cu") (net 7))
 (segment (start 64.62 86.255) (end 64.62 72.315) (width 0.2) (layer "F.Cu") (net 7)))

